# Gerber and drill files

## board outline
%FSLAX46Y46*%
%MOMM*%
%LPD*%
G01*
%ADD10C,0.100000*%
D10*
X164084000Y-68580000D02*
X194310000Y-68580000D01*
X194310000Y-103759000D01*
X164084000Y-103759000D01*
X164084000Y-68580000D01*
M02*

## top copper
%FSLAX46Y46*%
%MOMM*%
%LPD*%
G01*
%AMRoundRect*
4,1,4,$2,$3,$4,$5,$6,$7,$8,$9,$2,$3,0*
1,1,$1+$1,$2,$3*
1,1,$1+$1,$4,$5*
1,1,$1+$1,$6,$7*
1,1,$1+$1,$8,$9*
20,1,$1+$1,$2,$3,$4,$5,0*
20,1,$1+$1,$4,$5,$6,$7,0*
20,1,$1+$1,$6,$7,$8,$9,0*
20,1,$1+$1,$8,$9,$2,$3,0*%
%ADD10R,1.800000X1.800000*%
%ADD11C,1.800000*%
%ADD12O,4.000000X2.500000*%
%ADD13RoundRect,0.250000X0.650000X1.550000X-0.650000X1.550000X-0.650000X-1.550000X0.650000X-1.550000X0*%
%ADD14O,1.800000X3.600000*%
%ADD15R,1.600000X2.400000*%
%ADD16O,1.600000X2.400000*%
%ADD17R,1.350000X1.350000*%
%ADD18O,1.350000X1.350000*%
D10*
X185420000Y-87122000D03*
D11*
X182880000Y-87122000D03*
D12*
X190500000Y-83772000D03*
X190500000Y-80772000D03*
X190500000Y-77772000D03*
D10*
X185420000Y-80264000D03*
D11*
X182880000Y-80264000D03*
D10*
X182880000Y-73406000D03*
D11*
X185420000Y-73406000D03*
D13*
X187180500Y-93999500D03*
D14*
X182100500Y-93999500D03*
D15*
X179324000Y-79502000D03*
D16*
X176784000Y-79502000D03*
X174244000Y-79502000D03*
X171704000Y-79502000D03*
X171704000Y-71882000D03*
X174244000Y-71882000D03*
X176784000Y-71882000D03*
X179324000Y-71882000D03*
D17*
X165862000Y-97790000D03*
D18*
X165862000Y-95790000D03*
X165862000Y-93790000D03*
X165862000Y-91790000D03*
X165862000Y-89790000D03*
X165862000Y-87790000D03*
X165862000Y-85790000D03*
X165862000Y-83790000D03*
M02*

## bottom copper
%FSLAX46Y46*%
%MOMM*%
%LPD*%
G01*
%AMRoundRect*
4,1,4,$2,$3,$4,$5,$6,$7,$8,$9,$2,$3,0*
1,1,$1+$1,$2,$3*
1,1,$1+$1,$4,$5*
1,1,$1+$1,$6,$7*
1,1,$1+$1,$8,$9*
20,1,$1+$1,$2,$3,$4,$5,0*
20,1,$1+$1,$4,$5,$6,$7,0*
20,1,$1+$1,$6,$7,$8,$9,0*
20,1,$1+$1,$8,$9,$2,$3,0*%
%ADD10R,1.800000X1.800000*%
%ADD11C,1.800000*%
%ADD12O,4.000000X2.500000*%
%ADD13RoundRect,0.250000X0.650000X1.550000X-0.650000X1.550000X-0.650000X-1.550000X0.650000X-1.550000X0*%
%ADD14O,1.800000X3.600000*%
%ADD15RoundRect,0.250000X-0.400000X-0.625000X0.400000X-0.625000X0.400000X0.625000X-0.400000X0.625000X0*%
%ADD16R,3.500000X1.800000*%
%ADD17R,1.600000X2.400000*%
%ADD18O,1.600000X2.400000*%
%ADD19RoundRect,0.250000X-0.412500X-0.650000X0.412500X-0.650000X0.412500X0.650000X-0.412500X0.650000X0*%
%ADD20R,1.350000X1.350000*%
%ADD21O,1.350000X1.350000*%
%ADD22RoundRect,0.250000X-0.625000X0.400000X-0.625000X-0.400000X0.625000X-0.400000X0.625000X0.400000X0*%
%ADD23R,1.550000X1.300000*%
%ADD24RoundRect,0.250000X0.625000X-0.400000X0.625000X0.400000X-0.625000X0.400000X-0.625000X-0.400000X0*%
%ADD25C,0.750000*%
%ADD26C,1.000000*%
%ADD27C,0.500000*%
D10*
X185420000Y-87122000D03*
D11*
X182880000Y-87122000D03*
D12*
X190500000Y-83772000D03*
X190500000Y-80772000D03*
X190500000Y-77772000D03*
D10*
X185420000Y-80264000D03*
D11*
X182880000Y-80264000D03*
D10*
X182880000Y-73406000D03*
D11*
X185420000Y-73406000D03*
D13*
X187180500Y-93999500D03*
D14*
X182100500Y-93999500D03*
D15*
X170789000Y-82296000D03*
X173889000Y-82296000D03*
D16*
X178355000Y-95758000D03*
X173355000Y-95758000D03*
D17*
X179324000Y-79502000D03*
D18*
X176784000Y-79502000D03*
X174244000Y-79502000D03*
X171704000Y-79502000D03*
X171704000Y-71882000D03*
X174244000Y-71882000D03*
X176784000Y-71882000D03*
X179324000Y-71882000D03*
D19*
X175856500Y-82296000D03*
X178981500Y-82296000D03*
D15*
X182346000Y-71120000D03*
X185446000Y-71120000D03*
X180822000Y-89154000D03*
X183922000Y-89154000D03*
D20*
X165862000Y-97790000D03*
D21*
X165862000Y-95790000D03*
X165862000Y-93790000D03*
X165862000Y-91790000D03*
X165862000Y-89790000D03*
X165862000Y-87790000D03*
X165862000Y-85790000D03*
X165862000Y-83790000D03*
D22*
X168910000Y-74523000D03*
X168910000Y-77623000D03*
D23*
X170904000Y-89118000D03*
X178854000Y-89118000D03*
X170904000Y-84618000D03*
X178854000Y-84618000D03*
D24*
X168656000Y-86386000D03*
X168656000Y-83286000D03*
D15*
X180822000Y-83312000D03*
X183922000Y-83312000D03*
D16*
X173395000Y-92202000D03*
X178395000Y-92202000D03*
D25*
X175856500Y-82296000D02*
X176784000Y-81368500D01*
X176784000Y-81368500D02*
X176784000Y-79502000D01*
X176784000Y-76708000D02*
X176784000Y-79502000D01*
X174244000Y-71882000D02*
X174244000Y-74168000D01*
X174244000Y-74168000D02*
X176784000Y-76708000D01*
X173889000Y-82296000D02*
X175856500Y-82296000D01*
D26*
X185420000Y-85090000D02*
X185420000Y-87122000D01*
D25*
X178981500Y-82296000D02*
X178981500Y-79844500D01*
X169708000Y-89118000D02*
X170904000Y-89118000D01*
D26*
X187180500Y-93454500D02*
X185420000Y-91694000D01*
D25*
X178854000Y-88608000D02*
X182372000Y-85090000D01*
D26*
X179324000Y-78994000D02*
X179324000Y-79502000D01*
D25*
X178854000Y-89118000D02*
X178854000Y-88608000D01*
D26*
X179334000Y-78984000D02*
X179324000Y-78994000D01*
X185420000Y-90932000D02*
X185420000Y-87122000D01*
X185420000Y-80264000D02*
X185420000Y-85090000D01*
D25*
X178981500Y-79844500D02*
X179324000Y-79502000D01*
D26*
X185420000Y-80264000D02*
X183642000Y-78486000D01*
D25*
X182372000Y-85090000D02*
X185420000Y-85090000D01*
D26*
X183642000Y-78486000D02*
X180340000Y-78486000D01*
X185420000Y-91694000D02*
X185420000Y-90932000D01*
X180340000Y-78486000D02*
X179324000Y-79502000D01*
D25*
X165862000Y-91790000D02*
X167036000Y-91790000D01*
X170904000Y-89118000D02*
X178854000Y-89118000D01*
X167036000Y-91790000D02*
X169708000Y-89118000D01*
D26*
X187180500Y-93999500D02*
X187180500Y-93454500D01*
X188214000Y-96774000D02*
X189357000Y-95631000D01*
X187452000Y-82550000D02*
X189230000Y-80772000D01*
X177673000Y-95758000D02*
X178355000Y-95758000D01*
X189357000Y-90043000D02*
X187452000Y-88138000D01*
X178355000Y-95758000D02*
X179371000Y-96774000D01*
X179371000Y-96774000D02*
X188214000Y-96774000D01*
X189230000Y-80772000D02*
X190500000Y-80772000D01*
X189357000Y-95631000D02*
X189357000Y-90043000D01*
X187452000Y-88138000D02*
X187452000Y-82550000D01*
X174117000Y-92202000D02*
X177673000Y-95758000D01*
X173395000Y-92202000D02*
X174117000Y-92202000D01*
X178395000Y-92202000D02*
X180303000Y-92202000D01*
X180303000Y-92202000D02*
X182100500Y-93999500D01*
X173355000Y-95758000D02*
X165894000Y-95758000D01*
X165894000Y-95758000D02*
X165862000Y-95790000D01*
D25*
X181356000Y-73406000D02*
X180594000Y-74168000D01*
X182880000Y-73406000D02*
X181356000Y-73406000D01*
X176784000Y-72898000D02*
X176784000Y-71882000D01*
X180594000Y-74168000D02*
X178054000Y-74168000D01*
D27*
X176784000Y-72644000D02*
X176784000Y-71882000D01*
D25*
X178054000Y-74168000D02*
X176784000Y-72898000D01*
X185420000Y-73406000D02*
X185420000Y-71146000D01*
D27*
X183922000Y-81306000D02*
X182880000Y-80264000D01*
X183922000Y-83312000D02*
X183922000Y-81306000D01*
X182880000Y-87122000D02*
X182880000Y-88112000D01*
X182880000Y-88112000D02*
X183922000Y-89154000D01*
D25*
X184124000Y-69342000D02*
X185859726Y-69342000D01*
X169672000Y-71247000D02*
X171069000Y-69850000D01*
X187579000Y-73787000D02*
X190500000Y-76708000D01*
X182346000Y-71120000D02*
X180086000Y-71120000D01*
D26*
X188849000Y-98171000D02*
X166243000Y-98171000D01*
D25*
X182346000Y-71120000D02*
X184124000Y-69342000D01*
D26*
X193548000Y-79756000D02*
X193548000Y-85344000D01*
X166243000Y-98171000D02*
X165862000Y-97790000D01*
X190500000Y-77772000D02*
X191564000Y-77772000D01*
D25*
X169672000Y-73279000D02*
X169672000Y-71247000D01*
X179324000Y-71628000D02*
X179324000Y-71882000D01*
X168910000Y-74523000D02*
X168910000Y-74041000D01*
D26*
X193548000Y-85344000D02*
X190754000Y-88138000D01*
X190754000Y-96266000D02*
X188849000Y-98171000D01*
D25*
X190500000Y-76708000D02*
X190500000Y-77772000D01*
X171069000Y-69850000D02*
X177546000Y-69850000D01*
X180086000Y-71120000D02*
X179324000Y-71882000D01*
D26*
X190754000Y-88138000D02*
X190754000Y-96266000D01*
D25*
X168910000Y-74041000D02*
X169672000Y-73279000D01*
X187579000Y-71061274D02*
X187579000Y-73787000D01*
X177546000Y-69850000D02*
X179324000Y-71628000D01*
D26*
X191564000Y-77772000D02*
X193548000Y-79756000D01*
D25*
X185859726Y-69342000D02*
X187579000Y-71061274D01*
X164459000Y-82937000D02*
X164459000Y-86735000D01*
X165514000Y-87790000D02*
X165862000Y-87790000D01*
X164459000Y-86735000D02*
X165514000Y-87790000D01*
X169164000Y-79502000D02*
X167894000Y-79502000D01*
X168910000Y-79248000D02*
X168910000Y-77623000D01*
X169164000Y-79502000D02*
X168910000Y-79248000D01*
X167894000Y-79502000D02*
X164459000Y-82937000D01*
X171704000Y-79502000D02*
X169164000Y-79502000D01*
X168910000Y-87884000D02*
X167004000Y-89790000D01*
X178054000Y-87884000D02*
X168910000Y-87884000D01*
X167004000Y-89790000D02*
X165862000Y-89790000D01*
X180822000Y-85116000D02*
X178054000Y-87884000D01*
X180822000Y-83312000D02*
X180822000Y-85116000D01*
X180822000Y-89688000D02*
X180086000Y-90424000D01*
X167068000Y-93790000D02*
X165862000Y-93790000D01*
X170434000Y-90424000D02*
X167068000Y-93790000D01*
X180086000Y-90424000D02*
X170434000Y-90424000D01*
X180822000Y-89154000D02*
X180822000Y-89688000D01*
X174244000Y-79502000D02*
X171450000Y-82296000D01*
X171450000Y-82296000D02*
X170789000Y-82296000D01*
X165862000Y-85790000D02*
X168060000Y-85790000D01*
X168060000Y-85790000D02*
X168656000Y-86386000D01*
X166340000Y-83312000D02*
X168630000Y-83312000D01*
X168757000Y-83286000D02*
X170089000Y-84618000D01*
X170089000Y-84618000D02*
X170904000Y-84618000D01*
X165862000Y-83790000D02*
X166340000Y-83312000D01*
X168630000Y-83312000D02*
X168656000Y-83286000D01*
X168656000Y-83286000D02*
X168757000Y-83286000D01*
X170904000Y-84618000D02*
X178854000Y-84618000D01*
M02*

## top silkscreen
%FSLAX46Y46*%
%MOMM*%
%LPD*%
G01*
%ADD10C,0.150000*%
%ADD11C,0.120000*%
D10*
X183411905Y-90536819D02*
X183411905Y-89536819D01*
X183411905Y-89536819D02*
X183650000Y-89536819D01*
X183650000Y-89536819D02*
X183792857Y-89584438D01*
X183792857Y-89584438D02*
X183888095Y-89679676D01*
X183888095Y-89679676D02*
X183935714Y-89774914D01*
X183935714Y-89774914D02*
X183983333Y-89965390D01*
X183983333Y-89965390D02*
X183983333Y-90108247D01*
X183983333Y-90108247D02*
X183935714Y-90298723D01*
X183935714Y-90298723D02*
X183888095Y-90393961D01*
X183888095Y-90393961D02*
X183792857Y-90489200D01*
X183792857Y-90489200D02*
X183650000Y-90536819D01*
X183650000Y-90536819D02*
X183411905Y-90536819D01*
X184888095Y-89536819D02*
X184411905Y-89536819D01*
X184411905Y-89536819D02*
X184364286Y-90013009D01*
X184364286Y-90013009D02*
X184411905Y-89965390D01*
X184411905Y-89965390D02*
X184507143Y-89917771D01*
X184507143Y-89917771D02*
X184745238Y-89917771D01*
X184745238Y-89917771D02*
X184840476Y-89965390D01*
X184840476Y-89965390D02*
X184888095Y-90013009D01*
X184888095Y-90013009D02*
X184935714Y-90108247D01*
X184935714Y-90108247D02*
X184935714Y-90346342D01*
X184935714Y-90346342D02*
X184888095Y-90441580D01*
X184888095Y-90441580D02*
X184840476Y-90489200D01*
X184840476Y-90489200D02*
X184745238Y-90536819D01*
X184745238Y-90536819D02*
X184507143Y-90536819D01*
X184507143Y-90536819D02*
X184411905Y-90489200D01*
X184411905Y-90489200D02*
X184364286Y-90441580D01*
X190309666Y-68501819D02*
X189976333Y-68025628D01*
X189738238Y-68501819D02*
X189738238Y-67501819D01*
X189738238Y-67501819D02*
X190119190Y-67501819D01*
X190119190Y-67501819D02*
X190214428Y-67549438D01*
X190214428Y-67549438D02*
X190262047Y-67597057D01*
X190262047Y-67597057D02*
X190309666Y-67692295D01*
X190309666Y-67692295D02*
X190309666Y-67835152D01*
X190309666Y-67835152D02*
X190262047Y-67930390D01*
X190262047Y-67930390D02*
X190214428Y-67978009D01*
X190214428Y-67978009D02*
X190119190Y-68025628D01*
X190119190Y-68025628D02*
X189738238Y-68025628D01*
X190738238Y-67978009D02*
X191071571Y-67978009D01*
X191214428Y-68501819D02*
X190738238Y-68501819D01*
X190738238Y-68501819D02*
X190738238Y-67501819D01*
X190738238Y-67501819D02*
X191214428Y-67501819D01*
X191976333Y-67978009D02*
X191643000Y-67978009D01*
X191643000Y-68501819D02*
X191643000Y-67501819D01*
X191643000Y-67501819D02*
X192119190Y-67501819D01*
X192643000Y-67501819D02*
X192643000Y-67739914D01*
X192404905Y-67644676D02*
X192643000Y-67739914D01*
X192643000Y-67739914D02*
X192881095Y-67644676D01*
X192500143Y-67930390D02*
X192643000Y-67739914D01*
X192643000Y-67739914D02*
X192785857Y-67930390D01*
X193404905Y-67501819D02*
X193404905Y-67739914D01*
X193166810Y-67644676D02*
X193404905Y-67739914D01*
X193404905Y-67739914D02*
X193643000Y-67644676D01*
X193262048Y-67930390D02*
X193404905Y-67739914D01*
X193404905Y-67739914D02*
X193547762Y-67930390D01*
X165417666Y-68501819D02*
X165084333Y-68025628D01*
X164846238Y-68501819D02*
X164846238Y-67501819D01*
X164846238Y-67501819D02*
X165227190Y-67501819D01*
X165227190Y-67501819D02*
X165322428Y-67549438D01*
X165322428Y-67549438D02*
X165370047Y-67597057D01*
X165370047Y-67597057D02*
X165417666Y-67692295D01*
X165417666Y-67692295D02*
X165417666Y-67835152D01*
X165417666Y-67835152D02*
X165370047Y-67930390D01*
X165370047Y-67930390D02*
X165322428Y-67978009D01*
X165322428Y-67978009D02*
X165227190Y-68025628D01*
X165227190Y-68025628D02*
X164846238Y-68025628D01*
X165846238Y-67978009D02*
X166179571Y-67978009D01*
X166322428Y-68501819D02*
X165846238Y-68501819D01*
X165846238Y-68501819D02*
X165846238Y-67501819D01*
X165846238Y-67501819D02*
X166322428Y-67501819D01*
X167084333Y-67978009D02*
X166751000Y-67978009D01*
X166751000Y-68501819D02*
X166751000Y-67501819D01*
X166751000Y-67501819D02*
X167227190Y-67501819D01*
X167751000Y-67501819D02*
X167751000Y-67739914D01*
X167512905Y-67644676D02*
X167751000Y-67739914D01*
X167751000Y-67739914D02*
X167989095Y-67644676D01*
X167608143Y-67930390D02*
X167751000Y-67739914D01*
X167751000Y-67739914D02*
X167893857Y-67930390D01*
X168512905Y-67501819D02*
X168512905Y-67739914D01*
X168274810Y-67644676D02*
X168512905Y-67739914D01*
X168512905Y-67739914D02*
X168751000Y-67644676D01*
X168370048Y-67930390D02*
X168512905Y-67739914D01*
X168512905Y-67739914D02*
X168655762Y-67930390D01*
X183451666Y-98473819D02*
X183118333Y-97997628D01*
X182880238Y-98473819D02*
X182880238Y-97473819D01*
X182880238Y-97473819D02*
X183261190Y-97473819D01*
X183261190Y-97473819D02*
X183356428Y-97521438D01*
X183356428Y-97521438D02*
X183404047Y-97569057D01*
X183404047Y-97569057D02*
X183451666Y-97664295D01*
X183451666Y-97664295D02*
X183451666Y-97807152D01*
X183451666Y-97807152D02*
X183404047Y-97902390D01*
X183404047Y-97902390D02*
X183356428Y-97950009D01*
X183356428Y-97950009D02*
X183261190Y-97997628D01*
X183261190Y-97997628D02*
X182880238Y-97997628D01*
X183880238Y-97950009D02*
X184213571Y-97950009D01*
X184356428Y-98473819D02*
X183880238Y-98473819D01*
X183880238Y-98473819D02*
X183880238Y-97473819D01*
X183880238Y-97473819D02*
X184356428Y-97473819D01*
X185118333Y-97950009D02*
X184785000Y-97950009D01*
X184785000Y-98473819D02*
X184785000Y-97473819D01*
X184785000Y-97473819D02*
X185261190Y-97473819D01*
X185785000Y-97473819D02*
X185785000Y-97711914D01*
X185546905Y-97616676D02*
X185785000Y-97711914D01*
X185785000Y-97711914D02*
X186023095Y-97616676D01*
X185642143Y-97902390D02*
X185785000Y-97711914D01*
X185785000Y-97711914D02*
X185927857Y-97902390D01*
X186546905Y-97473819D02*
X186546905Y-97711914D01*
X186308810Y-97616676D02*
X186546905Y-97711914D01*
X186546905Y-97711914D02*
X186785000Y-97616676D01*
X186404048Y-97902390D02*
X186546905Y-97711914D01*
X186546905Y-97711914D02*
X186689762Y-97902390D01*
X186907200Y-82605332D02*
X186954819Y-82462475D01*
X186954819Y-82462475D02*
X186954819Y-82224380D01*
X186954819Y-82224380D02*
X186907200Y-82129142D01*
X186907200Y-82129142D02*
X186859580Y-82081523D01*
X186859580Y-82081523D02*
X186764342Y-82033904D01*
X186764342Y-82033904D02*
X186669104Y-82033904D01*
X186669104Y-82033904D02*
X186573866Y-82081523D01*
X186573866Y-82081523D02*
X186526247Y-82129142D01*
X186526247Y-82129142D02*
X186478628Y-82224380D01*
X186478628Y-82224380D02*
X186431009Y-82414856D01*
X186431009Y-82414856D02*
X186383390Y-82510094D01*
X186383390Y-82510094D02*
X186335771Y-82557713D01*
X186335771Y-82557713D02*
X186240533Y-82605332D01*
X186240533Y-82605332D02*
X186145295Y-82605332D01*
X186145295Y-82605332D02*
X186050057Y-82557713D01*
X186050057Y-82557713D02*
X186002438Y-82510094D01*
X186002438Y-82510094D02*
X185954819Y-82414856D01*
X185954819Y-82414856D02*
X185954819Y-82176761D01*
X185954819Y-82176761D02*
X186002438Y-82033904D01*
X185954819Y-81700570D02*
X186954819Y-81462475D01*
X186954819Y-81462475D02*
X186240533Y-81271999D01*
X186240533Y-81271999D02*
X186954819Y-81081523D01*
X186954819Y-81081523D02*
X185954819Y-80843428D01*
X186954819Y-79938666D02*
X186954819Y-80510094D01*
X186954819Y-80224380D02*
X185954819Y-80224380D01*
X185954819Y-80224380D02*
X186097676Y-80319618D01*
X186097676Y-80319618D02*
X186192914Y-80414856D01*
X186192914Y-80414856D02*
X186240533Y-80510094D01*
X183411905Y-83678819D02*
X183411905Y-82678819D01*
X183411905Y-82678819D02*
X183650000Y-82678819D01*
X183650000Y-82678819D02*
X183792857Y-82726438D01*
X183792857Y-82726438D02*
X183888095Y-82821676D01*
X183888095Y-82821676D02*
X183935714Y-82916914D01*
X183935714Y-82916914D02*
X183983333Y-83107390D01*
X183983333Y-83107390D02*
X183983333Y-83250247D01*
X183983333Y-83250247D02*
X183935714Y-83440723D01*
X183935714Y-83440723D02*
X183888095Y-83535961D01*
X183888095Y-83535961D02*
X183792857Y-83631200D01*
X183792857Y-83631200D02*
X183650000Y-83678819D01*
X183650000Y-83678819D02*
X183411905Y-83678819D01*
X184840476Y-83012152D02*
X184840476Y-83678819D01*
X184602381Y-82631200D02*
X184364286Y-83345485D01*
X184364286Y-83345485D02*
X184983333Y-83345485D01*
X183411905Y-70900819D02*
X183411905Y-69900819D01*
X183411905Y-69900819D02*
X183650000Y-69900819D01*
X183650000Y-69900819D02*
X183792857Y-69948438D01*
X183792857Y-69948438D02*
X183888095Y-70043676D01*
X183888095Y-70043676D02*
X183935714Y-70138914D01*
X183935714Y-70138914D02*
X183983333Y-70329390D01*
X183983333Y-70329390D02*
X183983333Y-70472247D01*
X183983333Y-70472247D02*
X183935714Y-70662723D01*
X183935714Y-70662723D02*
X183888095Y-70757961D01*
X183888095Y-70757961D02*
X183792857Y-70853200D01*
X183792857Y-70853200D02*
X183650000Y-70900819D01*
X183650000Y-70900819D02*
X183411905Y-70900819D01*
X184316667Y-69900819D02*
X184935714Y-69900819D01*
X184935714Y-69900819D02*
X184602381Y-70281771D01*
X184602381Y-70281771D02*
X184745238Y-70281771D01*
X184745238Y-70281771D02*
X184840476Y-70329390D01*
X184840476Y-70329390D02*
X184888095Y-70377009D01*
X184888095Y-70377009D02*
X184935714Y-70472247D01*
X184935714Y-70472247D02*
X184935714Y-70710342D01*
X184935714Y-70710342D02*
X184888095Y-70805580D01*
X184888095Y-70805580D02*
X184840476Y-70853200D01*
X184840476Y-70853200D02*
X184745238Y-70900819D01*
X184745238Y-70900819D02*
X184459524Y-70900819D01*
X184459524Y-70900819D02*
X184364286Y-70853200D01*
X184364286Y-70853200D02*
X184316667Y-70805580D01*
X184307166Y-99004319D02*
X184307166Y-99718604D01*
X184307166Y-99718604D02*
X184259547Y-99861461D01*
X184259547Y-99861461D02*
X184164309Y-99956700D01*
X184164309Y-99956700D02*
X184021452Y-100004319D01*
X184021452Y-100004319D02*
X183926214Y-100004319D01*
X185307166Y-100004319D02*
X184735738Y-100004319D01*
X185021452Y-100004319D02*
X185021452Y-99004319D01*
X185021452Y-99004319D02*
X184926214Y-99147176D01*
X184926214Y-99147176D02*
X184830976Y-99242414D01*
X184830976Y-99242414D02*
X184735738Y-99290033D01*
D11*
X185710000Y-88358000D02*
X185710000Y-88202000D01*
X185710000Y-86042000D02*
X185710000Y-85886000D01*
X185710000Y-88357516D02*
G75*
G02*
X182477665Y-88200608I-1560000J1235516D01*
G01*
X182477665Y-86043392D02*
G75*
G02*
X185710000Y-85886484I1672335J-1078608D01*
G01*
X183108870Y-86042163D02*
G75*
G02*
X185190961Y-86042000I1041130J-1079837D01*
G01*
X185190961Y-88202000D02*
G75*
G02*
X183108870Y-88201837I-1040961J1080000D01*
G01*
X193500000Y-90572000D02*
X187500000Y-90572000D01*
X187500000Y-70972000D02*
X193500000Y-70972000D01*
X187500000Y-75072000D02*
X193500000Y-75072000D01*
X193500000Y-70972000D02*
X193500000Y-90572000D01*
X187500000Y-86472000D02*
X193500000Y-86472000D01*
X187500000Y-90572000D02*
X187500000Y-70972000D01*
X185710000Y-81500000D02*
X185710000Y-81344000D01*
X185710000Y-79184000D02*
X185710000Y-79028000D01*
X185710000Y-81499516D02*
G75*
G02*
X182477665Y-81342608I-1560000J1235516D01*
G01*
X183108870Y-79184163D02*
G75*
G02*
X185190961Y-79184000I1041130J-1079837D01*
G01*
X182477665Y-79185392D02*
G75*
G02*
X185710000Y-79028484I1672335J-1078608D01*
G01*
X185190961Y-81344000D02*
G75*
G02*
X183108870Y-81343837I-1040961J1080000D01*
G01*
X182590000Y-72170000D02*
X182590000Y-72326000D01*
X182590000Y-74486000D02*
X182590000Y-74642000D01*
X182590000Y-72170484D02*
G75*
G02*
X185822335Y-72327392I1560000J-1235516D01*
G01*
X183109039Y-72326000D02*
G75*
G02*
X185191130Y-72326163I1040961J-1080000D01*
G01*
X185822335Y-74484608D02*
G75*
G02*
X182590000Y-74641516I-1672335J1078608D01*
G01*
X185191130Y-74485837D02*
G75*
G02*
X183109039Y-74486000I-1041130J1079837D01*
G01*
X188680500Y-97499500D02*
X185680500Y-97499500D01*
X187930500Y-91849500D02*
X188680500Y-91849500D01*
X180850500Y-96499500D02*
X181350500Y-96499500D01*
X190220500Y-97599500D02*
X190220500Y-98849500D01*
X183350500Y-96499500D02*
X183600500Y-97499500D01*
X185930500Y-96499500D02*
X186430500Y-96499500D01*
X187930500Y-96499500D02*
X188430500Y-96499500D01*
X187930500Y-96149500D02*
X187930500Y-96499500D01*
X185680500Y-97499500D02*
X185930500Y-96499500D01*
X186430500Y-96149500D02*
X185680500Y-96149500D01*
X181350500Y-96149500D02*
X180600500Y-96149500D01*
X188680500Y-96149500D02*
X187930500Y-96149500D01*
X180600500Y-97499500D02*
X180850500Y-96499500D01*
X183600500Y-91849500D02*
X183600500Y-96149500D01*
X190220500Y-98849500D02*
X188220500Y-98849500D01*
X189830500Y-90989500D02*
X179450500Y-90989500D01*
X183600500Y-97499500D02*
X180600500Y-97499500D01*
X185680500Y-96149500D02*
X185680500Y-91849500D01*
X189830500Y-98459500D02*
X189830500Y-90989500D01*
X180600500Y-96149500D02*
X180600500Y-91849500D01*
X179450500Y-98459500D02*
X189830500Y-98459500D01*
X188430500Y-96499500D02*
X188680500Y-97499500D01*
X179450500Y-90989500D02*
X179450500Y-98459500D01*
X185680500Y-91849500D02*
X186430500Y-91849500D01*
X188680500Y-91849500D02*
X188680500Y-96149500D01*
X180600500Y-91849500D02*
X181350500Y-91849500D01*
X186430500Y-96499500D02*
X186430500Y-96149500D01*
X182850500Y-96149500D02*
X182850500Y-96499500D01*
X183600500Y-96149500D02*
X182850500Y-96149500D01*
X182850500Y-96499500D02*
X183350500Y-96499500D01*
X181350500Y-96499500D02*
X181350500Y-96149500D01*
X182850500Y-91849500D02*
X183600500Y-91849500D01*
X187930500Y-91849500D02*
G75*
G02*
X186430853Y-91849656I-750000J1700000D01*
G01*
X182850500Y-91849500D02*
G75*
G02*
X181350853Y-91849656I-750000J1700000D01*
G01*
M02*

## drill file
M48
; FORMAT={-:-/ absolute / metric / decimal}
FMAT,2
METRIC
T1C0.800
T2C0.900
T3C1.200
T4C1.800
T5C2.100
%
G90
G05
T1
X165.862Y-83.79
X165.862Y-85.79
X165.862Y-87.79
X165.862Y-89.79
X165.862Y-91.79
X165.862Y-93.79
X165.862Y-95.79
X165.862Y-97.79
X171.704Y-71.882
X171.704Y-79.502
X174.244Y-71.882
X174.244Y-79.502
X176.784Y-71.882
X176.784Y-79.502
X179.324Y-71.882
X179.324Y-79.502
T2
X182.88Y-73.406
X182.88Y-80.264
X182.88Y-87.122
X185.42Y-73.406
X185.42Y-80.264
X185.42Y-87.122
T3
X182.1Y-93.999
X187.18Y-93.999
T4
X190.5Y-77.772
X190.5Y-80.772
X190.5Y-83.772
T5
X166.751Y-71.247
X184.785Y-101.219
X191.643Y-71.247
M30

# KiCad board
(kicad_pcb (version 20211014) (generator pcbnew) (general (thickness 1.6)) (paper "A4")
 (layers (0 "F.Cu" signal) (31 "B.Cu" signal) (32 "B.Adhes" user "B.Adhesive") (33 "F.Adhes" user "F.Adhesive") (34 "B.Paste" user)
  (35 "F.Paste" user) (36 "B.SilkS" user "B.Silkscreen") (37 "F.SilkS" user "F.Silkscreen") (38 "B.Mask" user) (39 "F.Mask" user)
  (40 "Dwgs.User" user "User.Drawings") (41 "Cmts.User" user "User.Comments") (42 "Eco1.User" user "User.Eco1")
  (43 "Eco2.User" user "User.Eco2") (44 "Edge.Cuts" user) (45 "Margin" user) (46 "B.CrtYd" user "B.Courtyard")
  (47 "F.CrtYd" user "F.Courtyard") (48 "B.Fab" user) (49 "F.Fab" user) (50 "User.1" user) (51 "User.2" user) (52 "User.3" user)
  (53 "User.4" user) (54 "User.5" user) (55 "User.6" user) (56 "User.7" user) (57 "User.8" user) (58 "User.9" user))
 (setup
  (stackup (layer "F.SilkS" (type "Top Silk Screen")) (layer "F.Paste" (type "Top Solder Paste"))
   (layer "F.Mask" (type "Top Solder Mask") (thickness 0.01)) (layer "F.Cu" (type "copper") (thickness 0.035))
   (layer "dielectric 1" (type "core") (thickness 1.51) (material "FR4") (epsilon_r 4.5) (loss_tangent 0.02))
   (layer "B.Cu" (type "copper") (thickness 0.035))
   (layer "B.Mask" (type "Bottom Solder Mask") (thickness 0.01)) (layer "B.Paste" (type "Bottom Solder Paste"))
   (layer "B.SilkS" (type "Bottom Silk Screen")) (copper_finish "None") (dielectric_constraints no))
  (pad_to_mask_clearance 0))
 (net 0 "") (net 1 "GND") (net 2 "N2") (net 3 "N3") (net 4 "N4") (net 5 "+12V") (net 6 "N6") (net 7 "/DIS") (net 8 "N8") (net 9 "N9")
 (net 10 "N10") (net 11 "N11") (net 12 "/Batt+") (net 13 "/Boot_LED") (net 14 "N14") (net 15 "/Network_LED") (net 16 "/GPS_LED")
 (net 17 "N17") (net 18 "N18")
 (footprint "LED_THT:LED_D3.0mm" (layer "F.Cu") (at 185.42 87.122 180)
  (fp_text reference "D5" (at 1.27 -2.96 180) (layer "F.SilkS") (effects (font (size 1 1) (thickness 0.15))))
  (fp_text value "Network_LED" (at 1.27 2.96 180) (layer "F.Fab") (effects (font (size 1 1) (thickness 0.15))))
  (fp_line (start -0.29 -1.236) (end -0.29 -1.08) (layer "F.SilkS") (width 0.12))
  (fp_line (start -0.29 1.08) (end -0.29 1.236) (layer "F.SilkS") (width 0.12))
  (fp_arc (start -0.29 -1.235516) (mid 1.366487 -1.987659) (end 2.942335 -1.078608) (layer "F.SilkS") (width 0.12))
  (fp_arc (start 2.942335 1.078608) (mid 1.366487 1.987659) (end -0.29 1.235516) (layer "F.SilkS") (width 0.12))
  (fp_arc (start 2.31113 1.079837) (mid 1.270117 1.5) (end 0.229039 1.08) (layer "F.SilkS") (width 0.12))
  (fp_arc (start 0.229039 -1.08) (mid 1.270117 -1.5) (end 2.31113 -1.079837) (layer "F.SilkS") (width 0.12))
  (pad "1" thru_hole rect (at 0 0 180) (size 1.8 1.8) (drill 0.9) (layers *.Cu *.Mask) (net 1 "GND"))
  (pad "2" thru_hole circle (at 2.54 0 180) (size 1.8 1.8) (drill 0.9) (layers *.Cu *.Mask) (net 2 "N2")))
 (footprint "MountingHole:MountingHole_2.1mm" (layer "F.Cu") (at 191.643 71.247)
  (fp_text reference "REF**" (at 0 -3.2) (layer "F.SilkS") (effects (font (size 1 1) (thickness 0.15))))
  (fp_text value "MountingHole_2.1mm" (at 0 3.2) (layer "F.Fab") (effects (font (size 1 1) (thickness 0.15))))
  (pad "" np_thru_hole circle (at 0 0) (size 2.1 2.1) (drill 2.1) (layers *.Cu *.Mask)))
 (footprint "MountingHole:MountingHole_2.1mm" (layer "F.Cu") (at 166.751 71.247)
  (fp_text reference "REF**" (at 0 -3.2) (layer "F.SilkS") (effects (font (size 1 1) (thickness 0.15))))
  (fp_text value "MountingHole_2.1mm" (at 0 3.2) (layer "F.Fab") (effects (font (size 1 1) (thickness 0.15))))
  (pad "" np_thru_hole circle (at 0 0) (size 2.1 2.1) (drill 2.1) (layers *.Cu *.Mask)))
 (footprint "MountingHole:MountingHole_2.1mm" (layer "F.Cu") (at 184.785 101.219)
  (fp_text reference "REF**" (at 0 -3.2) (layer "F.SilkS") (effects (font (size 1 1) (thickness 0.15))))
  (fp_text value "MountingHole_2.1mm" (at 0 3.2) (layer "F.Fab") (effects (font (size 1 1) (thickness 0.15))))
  (pad "" np_thru_hole circle (at 0 0) (size 2.1 2.1) (drill 2.1) (layers *.Cu *.Mask)))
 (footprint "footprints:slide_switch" (layer "F.Cu") (at 190.5 80.772 90) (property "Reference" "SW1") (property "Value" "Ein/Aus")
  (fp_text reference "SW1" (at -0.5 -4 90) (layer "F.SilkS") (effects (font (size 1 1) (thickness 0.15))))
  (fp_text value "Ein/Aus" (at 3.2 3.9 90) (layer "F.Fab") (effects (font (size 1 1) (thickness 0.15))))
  (fp_line (start -9.8 3) (end -9.8 -3) (layer "F.SilkS") (width 0.12))
  (fp_line (start 9.8 -3) (end 9.8 3) (layer "F.SilkS") (width 0.12))
  (fp_line (start 5.7 -3) (end 5.7 3) (layer "F.SilkS") (width 0.12))
  (fp_line (start 9.8 3) (end -9.8 3) (layer "F.SilkS") (width 0.12))
  (fp_line (start -5.7 -3) (end -5.7 3) (layer "F.SilkS") (width 0.12))
  (fp_line (start -9.8 -3) (end 9.8 -3) (layer "F.SilkS") (width 0.12))
  (pad "1" thru_hole oval (at -3 0 90) (size 2.5 4) (drill 1.8) (layers *.Cu *.Mask) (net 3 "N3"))
  (pad "2" thru_hole oval (at 0 0 90) (size 2.5 4) (drill 1.8) (layers *.Cu *.Mask) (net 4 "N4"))
  (pad "3" thru_hole oval (at 3 0 90) (size 2.5 4) (drill 1.8) (layers *.Cu *.Mask) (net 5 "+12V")))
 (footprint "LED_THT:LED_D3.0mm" (layer "F.Cu") (at 185.42 80.264 180) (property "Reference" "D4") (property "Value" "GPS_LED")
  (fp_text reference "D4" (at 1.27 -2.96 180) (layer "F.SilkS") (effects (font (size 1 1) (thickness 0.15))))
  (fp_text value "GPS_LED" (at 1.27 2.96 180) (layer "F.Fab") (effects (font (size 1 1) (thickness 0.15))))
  (fp_line (start -0.29 -1.236) (end -0.29 -1.08) (layer "F.SilkS") (width 0.12))
  (fp_line (start -0.29 1.08) (end -0.29 1.236) (layer "F.SilkS") (width 0.12))
  (fp_arc (start -0.29 -1.235516) (mid 1.366487 -1.987659) (end 2.942335 -1.078608) (layer "F.SilkS") (width 0.12))
  (fp_arc (start 2.31113 1.079837) (mid 1.270117 1.5) (end 0.229039 1.08) (layer "F.SilkS") (width 0.12))
  (fp_arc (start 2.942335 1.078608) (mid 1.366487 1.987659) (end -0.29 1.235516) (layer "F.SilkS") (width 0.12))
  (fp_arc (start 0.229039 -1.08) (mid 1.270117 -1.5) (end 2.31113 -1.079837) (layer "F.SilkS") (width 0.12))
  (pad "1" thru_hole rect (at 0 0 180) (size 1.8 1.8) (drill 0.9) (layers *.Cu *.Mask) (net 1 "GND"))
  (pad "2" thru_hole circle (at 2.54 0 180) (size 1.8 1.8) (drill 0.9) (layers *.Cu *.Mask) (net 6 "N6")))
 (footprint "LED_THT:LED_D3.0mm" (layer "F.Cu") (at 182.88 73.406)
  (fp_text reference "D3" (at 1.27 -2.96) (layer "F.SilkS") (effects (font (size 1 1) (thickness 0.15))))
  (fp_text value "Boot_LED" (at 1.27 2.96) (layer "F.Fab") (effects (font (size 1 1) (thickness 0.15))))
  (fp_line (start -0.29 -1.236) (end -0.29 -1.08) (layer "F.SilkS") (width 0.12))
  (fp_line (start -0.29 1.08) (end -0.29 1.236) (layer "F.SilkS") (width 0.12))
  (fp_arc (start -0.29 -1.235516) (mid 1.366487 -1.987659) (end 2.942335 -1.078608) (layer "F.SilkS") (width 0.12))
  (fp_arc (start 0.229039 -1.08) (mid 1.270117 -1.5) (end 2.31113 -1.079837) (layer "F.SilkS") (width 0.12))
  (fp_arc (start 2.942335 1.078608) (mid 1.366487 1.987659) (end -0.29 1.235516) (layer "F.SilkS") (width 0.12))
  (fp_arc (start 2.31113 1.079837) (mid 1.270117 1.5) (end 0.229039 1.08) (layer "F.SilkS") (width 0.12))
  (pad "1" thru_hole rect (at 0 0) (size 1.8 1.8) (drill 0.9) (layers *.Cu *.Mask) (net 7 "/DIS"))
  (pad "2" thru_hole circle (at 2.54 0) (size 1.8 1.8) (drill 0.9) (layers *.Cu *.Mask) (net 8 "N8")))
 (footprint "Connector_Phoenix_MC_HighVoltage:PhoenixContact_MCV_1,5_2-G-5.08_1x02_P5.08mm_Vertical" (layer "F.Cu")
  (at 187.1805 93.9995 180) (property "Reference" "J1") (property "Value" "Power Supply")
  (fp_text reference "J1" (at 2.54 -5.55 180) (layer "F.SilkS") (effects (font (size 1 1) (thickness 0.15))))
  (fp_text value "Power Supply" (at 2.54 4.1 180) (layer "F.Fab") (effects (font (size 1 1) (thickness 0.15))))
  (fp_line (start -1.5 -3.5) (end 1.5 -3.5) (layer "F.SilkS") (width 0.12))
  (fp_line (start -0.75 2.15) (end -1.5 2.15) (layer "F.SilkS") (width 0.12))
  (fp_line (start 6.33 -2.5) (end 5.83 -2.5) (layer "F.SilkS") (width 0.12))
  (fp_line (start -3.04 -3.6) (end -3.04 -4.85) (layer "F.SilkS") (width 0.12))
  (fp_line (start 3.83 -2.5) (end 3.58 -3.5) (layer "F.SilkS") (width 0.12))
  (fp_line (start 1.25 -2.5) (end 0.75 -2.5) (layer "F.SilkS") (width 0.12))
  (fp_line (start -0.75 -2.5) (end -1.25 -2.5) (layer "F.SilkS") (width 0.12))
  (fp_line (start -0.75 -2.15) (end -0.75 -2.5) (layer "F.SilkS") (width 0.12))
  (fp_line (start 1.5 -3.5) (end 1.25 -2.5) (layer "F.SilkS") (width 0.12))
  (fp_line (start 0.75 -2.15) (end 1.5 -2.15) (layer "F.SilkS") (width 0.12))
  (fp_line (start 5.83 -2.15) (end 6.58 -2.15) (layer "F.SilkS") (width 0.12))
  (fp_line (start -1.5 -2.15) (end -0.75 -2.15) (layer "F.SilkS") (width 0.12))
  (fp_line (start 6.58 -3.5) (end 6.33 -2.5) (layer "F.SilkS") (width 0.12))
  (fp_line (start 3.58 2.15) (end 3.58 -2.15) (layer "F.SilkS") (width 0.12))
  (fp_line (start -3.04 -4.85) (end -1.04 -4.85) (layer "F.SilkS") (width 0.12))
  (fp_line (start -2.65 3.01) (end 7.73 3.01) (layer "F.SilkS") (width 0.12))
  (fp_line (start 3.58 -3.5) (end 6.58 -3.5) (layer "F.SilkS") (width 0.12))
  (fp_line (start 1.5 -2.15) (end 1.5 2.15) (layer "F.SilkS") (width 0.12))
  (fp_line (start -2.65 -4.46) (end -2.65 3.01) (layer "F.SilkS") (width 0.12))
  (fp_line (start 6.58 -2.15) (end 6.58 2.15) (layer "F.SilkS") (width 0.12))
  (fp_line (start 7.73 -4.46) (end -2.65 -4.46) (layer "F.SilkS") (width 0.12))
  (fp_line (start -1.25 -2.5) (end -1.5 -3.5) (layer "F.SilkS") (width 0.12))
  (fp_line (start 7.73 3.01) (end 7.73 -4.46) (layer "F.SilkS") (width 0.12))
  (fp_line (start 1.5 2.15) (end 0.75 2.15) (layer "F.SilkS") (width 0.12))
  (fp_line (start -1.5 2.15) (end -1.5 -2.15) (layer "F.SilkS") (width 0.12))
  (fp_line (start 6.58 2.15) (end 5.83 2.15) (layer "F.SilkS") (width 0.12))
  (fp_line (start 0.75 -2.5) (end 0.75 -2.15) (layer "F.SilkS") (width 0.12))
  (fp_line (start 4.33 -2.15) (end 4.33 -2.5) (layer "F.SilkS") (width 0.12))
  (fp_line (start 3.58 -2.15) (end 4.33 -2.15) (layer "F.SilkS") (width 0.12))
  (fp_line (start 4.33 -2.5) (end 3.83 -2.5) (layer "F.SilkS") (width 0.12))
  (fp_line (start 5.83 -2.5) (end 5.83 -2.15) (layer "F.SilkS") (width 0.12))
  (fp_line (start 4.33 2.15) (end 3.58 2.15) (layer "F.SilkS") (width 0.12))
  (fp_arc (start -0.75 2.15) (mid -0.000193 1.99191) (end 0.749647 2.149844) (layer "F.SilkS") (width 0.12))
  (fp_arc (start 4.33 2.15) (mid 5.079807 1.99191) (end 5.829647 2.149844) (layer "F.SilkS") (width 0.12))
  (pad "1" thru_hole roundrect (at 0 0 180) (size 1.8 3.6) (drill 1.2) (layers *.Cu *.Mask) (roundrect_rratio 0.1388888889) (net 1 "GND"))
  (pad "2" thru_hole oval (at 5.08 0 180) (size 1.8 3.6) (drill 1.2) (layers *.Cu *.Mask) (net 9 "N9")))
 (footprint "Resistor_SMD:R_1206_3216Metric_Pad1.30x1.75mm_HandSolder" (layer "B.Cu") (at 172.339 82.296) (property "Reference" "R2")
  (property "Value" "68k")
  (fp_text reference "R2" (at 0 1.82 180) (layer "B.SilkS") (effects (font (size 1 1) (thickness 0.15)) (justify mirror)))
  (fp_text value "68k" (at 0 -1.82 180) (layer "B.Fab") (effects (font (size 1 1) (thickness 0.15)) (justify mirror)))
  (pad "1" smd roundrect (at -1.55 0) (size 1.3 1.75) (layers "B.Cu" "B.Paste" "B.Mask") (roundrect_rratio 0.1923076923) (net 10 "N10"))
  (pad "2" smd roundrect (at 1.55 0) (size 1.3 1.75) (layers "B.Cu" "B.Paste" "B.Mask") (roundrect_rratio 0.1923076923) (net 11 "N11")))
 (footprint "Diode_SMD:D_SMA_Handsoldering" (layer "B.Cu") (at 175.855 95.758 180) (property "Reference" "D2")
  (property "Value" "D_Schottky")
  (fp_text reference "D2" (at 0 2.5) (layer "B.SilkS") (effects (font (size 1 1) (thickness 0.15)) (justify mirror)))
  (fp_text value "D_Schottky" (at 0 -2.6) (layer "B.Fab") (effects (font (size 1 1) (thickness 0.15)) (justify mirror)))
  (pad "1" smd rect (at -2.5 0 180) (size 3.5 1.8) (layers "B.Cu" "B.Paste" "B.Mask") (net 4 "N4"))
  (pad "2" smd rect (at 2.5 0 180) (size 3.5 1.8) (layers "B.Cu" "B.Paste" "B.Mask") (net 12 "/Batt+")))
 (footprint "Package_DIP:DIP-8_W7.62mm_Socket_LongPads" (layer "B.Cu") (at 179.324 79.502 90) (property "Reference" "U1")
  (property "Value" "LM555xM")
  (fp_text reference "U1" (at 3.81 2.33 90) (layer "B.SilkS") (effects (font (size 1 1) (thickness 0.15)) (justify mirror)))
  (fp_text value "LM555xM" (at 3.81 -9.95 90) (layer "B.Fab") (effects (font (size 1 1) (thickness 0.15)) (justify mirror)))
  (pad "1" thru_hole rect (at 0 0 90) (size 2.4 1.6) (drill 0.8) (layers *.Cu *.Mask) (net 1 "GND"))
  (pad "2" thru_hole oval (at 0 -2.54 90) (size 2.4 1.6) (drill 0.8) (layers *.Cu *.Mask) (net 11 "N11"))
  (pad "3" thru_hole oval (at 0 -5.08 90) (size 2.4 1.6) (drill 0.8) (layers *.Cu *.Mask) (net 10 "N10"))
  (pad "4" thru_hole oval (at 0 -7.62 90) (size 2.4 1.6) (drill 0.8) (layers *.Cu *.Mask) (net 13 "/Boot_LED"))
  (pad "5" thru_hole oval (at 7.62 -7.62 90) (size 2.4 1.6) (drill 0.8) (layers *.Cu *.Mask) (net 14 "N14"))
  (pad "6" thru_hole oval (at 7.62 -5.08 90) (size 2.4 1.6) (drill 0.8) (layers *.Cu *.Mask) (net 11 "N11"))
  (pad "7" thru_hole oval (at 7.62 -2.54 90) (size 2.4 1.6) (drill 0.8) (layers *.Cu *.Mask) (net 7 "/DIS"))
  (pad "8" thru_hole oval (at 7.62 0 90) (size 2.4 1.6) (drill 0.8) (layers *.Cu *.Mask) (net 5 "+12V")))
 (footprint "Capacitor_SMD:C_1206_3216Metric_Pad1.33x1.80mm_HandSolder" (layer "B.Cu") (at 177.419 82.296) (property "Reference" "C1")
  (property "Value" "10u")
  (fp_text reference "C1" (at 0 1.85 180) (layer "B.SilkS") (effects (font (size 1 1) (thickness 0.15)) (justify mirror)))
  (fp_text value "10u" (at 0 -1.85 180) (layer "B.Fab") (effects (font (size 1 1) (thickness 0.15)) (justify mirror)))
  (pad "1" smd roundrect (at -1.5625 0) (size 1.325 1.8) (layers "B.Cu" "B.Paste" "B.Mask") (roundrect_rratio 0.1886792453) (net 11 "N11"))
  (pad "2" smd roundrect (at 1.5625 0) (size 1.325 1.8) (layers "B.Cu" "B.Paste" "B.Mask") (roundrect_rratio 0.1886792453) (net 1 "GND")))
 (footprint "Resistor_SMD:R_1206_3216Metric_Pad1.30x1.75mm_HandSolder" (layer "B.Cu") (at 183.896 71.12)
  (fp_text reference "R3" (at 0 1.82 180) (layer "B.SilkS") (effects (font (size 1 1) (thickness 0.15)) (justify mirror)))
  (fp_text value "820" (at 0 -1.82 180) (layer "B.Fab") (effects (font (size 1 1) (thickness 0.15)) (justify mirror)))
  (pad "1" smd roundrect (at -1.55 0) (size 1.3 1.75) (layers "B.Cu" "B.Paste" "B.Mask") (roundrect_rratio 0.1923076923) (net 5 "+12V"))
  (pad "2" smd roundrect (at 1.55 0) (size 1.3 1.75) (layers "B.Cu" "B.Paste" "B.Mask") (roundrect_rratio 0.1923076923) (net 8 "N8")))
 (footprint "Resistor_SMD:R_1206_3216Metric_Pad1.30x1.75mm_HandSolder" (layer "B.Cu") (at 182.372 89.154)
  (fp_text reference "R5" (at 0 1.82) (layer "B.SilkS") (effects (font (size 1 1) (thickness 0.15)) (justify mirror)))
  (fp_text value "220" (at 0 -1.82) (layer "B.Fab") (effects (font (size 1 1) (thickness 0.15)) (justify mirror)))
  (pad "1" smd roundrect (at -1.55 0) (size 1.3 1.75) (layers "B.Cu" "B.Paste" "B.Mask") (roundrect_rratio 0.1923076923)
   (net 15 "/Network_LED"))
  (pad "2" smd roundrect (at 1.55 0) (size 1.3 1.75) (layers "B.Cu" "B.Paste" "B.Mask") (roundrect_rratio 0.1923076923) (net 2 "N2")))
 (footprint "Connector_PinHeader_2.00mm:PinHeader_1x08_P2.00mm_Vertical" (layer "B.Cu") (at 165.862 97.79)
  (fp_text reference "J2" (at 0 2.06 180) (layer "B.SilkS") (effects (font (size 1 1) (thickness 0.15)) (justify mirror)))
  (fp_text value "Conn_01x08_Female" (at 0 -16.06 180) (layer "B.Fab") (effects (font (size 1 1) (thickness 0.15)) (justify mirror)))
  (pad "1" thru_hole rect (at 0 0) (size 1.35 1.35) (drill 0.8) (layers *.Cu *.Mask) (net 5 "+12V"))
  (pad "2" thru_hole oval (at 0 -2) (size 1.35 1.35) (drill 0.8) (layers *.Cu *.Mask) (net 12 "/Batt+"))
  (pad "3" thru_hole oval (at 0 -4) (size 1.35 1.35) (drill 0.8) (layers *.Cu *.Mask) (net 15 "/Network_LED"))
  (pad "4" thru_hole oval (at 0 -6) (size 1.35 1.35) (drill 0.8) (layers *.Cu *.Mask) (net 1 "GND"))
  (pad "5" thru_hole oval (at 0 -8) (size 1.35 1.35) (drill 0.8) (layers *.Cu *.Mask) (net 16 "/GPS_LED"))
  (pad "6" thru_hole oval (at 0 -10) (size 1.35 1.35) (drill 0.8) (layers *.Cu *.Mask) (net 13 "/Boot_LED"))
  (pad "7" thru_hole oval (at 0 -12) (size 1.35 1.35) (drill 0.8) (layers *.Cu *.Mask) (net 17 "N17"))
  (pad "8" thru_hole oval (at 0 -14) (size 1.35 1.35) (drill 0.8) (layers *.Cu *.Mask) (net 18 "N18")))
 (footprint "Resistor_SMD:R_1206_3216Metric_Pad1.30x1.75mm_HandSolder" (layer "B.Cu") (at 168.91 76.073 -90)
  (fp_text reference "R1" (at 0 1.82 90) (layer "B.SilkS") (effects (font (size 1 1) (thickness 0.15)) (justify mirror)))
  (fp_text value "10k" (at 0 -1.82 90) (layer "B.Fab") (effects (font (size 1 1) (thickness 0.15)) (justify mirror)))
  (pad "1" smd roundrect (at -1.55 0 270) (size 1.3 1.75) (layers "B.Cu" "B.Paste" "B.Mask") (roundrect_rratio 0.1923076923) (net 5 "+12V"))
  (pad "2" smd roundrect (at 1.55 0 270) (size 1.3 1.75) (layers "B.Cu" "B.Paste" "B.Mask") (roundrect_rratio 0.1923076923)
   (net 13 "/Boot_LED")))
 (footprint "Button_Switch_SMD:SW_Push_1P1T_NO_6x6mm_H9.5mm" (layer "B.Cu") (at 174.879 86.868)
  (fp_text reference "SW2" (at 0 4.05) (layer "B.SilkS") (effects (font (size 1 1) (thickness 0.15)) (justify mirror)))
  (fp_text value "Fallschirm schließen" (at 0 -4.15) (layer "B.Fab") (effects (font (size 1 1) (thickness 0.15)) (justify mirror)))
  (pad "1" smd rect (at -3.975 2.25) (size 1.55 1.3) (layers "B.Cu" "B.Paste" "B.Mask") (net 1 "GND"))
  (pad "1" smd rect (at 3.975 2.25) (size 1.55 1.3) (layers "B.Cu" "B.Paste" "B.Mask") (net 1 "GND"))
  (pad "2" smd rect (at -3.975 -2.25) (size 1.55 1.3) (layers "B.Cu" "B.Paste" "B.Mask") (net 18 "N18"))
  (pad "2" smd rect (at 3.975 -2.25) (size 1.55 1.3) (layers "B.Cu" "B.Paste" "B.Mask") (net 18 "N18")))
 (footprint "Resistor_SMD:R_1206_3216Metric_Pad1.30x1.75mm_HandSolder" (layer "B.Cu") (at 168.656 84.836 90)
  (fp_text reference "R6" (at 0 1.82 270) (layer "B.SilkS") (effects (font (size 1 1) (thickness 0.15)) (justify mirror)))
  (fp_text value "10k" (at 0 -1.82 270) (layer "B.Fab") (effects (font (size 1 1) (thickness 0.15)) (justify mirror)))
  (pad "1" smd roundrect (at -1.55 0 90) (size 1.3 1.75) (layers "B.Cu" "B.Paste" "B.Mask") (roundrect_rratio 0.1923076923) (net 17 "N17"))
  (pad "2" smd roundrect (at 1.55 0 90) (size 1.3 1.75) (layers "B.Cu" "B.Paste" "B.Mask") (roundrect_rratio 0.1923076923) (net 18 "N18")))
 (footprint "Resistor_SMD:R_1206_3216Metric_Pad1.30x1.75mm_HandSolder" (layer "B.Cu") (at 182.372 83.312) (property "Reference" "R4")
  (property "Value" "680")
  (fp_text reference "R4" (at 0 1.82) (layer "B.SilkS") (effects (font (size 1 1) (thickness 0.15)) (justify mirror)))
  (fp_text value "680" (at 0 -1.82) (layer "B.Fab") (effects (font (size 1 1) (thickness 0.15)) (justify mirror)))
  (pad "1" smd roundrect (at -1.55 0) (size 1.3 1.75) (layers "B.Cu" "B.Paste" "B.Mask") (roundrect_rratio 0.1923076923) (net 16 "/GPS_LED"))
  (pad "2" smd roundrect (at 1.55 0) (size 1.3 1.75) (layers "B.Cu" "B.Paste" "B.Mask") (roundrect_rratio 0.1923076923) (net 6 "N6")))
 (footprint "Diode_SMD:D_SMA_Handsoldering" (layer "B.Cu") (at 175.895 92.202) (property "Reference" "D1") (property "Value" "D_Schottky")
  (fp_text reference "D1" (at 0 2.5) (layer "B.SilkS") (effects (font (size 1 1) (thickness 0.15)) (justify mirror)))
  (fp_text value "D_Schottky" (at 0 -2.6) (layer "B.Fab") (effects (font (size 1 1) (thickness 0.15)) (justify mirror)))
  (pad "1" smd rect (at -2.5 0) (size 3.5 1.8) (layers "B.Cu" "B.Paste" "B.Mask") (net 4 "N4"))
  (pad "2" smd rect (at 2.5 0) (size 3.5 1.8) (layers "B.Cu" "B.Paste" "B.Mask") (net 9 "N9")))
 (gr_rect (start 164.084 68.58) (end 194.31 103.759) (layer "Edge.Cuts") (width 0.1) (fill none))
 (segment (start 175.8565 82.296) (end 176.784 81.3685) (width 0.75) (layer "B.Cu") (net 11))
 (segment (start 176.784 81.3685) (end 176.784 79.502) (width 0.75) (layer "B.Cu") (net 11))
 (segment (start 176.784 76.708) (end 176.784 79.502) (width 0.75) (layer "B.Cu") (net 11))
 (segment (start 174.244 71.882) (end 174.244 74.168) (width 0.75) (layer "B.Cu") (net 11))
 (segment (start 174.244 74.168) (end 176.784 76.708) (width 0.75) (layer "B.Cu") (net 11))
 (segment (start 173.889 82.296) (end 175.8565 82.296) (width 0.75) (layer "B.Cu") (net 11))
 (segment (start 185.42 85.09) (end 185.42 87.122) (width 1) (layer "B.Cu") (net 1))
 (segment (start 178.9815 82.296) (end 178.9815 79.8445) (width 0.75) (layer "B.Cu") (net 1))
 (segment (start 169.708 89.118) (end 170.904 89.118) (width 0.75) (layer "B.Cu") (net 1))
 (segment (start 187.1805 93.4545) (end 185.42 91.694) (width 1) (layer "B.Cu") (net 1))
 (segment (start 178.854 88.608) (end 182.372 85.09) (width 0.75) (layer "B.Cu") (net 1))
 (segment (start 179.324 78.994) (end 179.324 79.502) (width 1) (layer "B.Cu") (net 1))
 (segment (start 178.854 89.118) (end 178.854 88.608) (width 0.75) (layer "B.Cu") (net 1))
 (segment (start 179.334 78.984) (end 179.324 78.994) (width 1) (layer "B.Cu") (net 1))
 (segment (start 185.42 90.932) (end 185.42 87.122) (width 1) (layer "B.Cu") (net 1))
 (segment (start 185.42 80.264) (end 185.42 85.09) (width 1) (layer "B.Cu") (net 1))
 (segment (start 178.9815 79.8445) (end 179.324 79.502) (width 0.75) (layer "B.Cu") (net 1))
 (segment (start 185.42 80.264) (end 183.642 78.486) (width 1) (layer "B.Cu") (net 1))
 (segment (start 182.372 85.09) (end 185.42 85.09) (width 0.75) (layer "B.Cu") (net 1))
 (segment (start 183.642 78.486) (end 180.34 78.486) (width 1) (layer "B.Cu") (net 1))
 (segment (start 185.42 91.694) (end 185.42 90.932) (width 1) (layer "B.Cu") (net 1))
 (segment (start 180.34 78.486) (end 179.324 79.502) (width 1) (layer "B.Cu") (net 1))
 (segment (start 165.862 91.79) (end 167.036 91.79) (width 0.75) (layer "B.Cu") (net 1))
 (segment (start 170.904 89.118) (end 178.854 89.118) (width 0.75) (layer "B.Cu") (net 1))
 (segment (start 167.036 91.79) (end 169.708 89.118) (width 0.75) (layer "B.Cu") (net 1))
 (segment (start 187.1805 93.9995) (end 187.1805 93.4545) (width 1) (layer "B.Cu") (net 1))
 (segment (start 188.214 96.774) (end 189.357 95.631) (width 1) (layer "B.Cu") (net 4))
 (segment (start 187.452 82.55) (end 189.23 80.772) (width 1) (layer "B.Cu") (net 4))
 (segment (start 177.673 95.758) (end 178.355 95.758) (width 1) (layer "B.Cu") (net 4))
 (segment (start 189.357 90.043) (end 187.452 88.138) (width 1) (layer "B.Cu") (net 4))
 (segment (start 178.355 95.758) (end 179.371 96.774) (width 1) (layer "B.Cu") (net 4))
 (segment (start 179.371 96.774) (end 188.214 96.774) (width 1) (layer "B.Cu") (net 4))
 (segment (start 189.23 80.772) (end 190.5 80.772) (width 1) (layer "B.Cu") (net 4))
 (segment (start 189.357 95.631) (end 189.357 90.043) (width 1) (layer "B.Cu") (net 4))
 (segment (start 187.452 88.138) (end 187.452 82.55) (width 1) (layer "B.Cu") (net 4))
 (segment (start 174.117 92.202) (end 177.673 95.758) (width 1) (layer "B.Cu") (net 4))
 (segment (start 173.395 92.202) (end 174.117 92.202) (width 1) (layer "B.Cu") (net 4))
 (segment (start 178.395 92.202) (end 180.303 92.202) (width 1) (layer "B.Cu") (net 9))
 (segment (start 180.303 92.202) (end 182.1005 93.9995) (width 1) (layer "B.Cu") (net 9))
 (segment (start 173.355 95.758) (end 165.894 95.758) (width 1) (layer "B.Cu") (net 12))
 (segment (start 165.894 95.758) (end 165.862 95.79) (width 1) (layer "B.Cu") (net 12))
 (segment (start 181.356 73.406) (end 180.594 74.168) (width 0.75) (layer "B.Cu") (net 7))
 (segment (start 182.88 73.406) (end 181.356 73.406) (width 0.75) (layer "B.Cu") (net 7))
 (segment (start 176.784 72.898) (end 176.784 71.882) (width 0.75) (layer "B.Cu") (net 7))
 (segment (start 180.594 74.168) (end 178.054 74.168) (width 0.75) (layer "B.Cu") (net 7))
 (segment (start 176.784 72.644) (end 176.784 71.882) (width 0.5) (layer "B.Cu") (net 7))
 (segment (start 178.054 74.168) (end 176.784 72.898) (width 0.75) (layer "B.Cu") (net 7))
 (segment (start 185.42 73.406) (end 185.42 71.146) (width 0.75) (layer "B.Cu") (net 8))
 (segment (start 183.922 81.306) (end 182.88 80.264) (width 0.5) (layer "B.Cu") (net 6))
 (segment (start 183.922 83.312) (end 183.922 81.306) (width 0.5) (layer "B.Cu") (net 6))
 (segment (start 182.88 87.122) (end 182.88 88.112) (width 0.5) (layer "B.Cu") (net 2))
 (segment (start 182.88 88.112) (end 183.922 89.154) (width 0.5) (layer "B.Cu") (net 2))
 (segment (start 184.124 69.342) (end 185.859726 69.342) (width 0.75) (layer "B.Cu") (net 5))
 (segment (start 169.672 71.247) (end 171.069 69.85) (width 0.75) (layer "B.Cu") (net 5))
 (segment (start 187.579 73.787) (end 190.5 76.708) (width 0.75) (layer "B.Cu") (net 5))
 (segment (start 182.346 71.12) (end 180.086 71.12) (width 0.75) (layer "B.Cu") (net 5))
 (segment (start 188.849 98.171) (end 166.243 98.171) (width 1) (layer "B.Cu") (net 5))
 (segment (start 182.346 71.12) (end 184.124 69.342) (width 0.75) (layer "B.Cu") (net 5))
 (segment (start 193.548 79.756) (end 193.548 85.344) (width 1) (layer "B.Cu") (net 5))
 (segment (start 166.243 98.171) (end 165.862 97.79) (width 1) (layer "B.Cu") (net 5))
 (segment (start 190.5 77.772) (end 191.564 77.772) (width 1) (layer "B.Cu") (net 5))
 (segment (start 169.672 73.279) (end 169.672 71.247) (width 0.75) (layer "B.Cu") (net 5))
 (segment (start 179.324 71.628) (end 179.324 71.882) (width 0.75) (layer "B.Cu") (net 5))
 (segment (start 168.91 74.523) (end 168.91 74.041) (width 0.75) (layer "B.Cu") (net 5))
 (segment (start 193.548 85.344) (end 190.754 88.138) (width 1) (layer "B.Cu") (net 5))
 (segment (start 190.754 96.266) (end 188.849 98.171) (width 1) (layer "B.Cu") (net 5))
 (segment (start 190.5 76.708) (end 190.5 77.772) (width 0.75) (layer "B.Cu") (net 5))
 (segment (start 171.069 69.85) (end 177.546 69.85) (width 0.75) (layer "B.Cu") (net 5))
 (segment (start 180.086 71.12) (end 179.324 71.882) (width 0.75) (layer "B.Cu") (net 5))
 (segment (start 190.754 88.138) (end 190.754 96.266) (width 1) (layer "B.Cu") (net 5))
 (segment (start 168.91 74.041) (end 169.672 73.279) (width 0.75) (layer "B.Cu") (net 5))
 (segment (start 187.579 71.061274) (end 187.579 73.787) (width 0.75) (layer "B.Cu") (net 5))
 (segment (start 177.546 69.85) (end 179.324 71.628) (width 0.75) (layer "B.Cu") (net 5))
 (segment (start 191.564 77.772) (end 193.548 79.756) (width 1) (layer "B.Cu") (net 5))
 (segment (start 185.859726 69.342) (end 187.579 71.061274) (width 0.75) (layer "B.Cu") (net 5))
 (segment (start 164.459 82.937) (end 164.459 86.735) (width 0.75) (layer "B.Cu") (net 13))
 (segment (start 165.514 87.79) (end 165.862 87.79) (width 0.75) (layer "B.Cu") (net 13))
 (segment (start 164.459 86.735) (end 165.514 87.79) (width 0.75) (layer "B.Cu") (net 13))
 (segment (start 169.164 79.502) (end 167.894 79.502) (width 0.75) (layer "B.Cu") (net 13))
 (segment (start 168.91 79.248) (end 168.91 77.623) (width 0.75) (layer "B.Cu") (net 13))
 (segment (start 169.164 79.502) (end 168.91 79.248) (width 0.75) (layer "B.Cu") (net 13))
 (segment (start 167.894 79.502) (end 164.459 82.937) (width 0.75) (layer "B.Cu") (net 13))
 (segment (start 171.704 79.502) (end 169.164 79.502) (width 0.75) (layer "B.Cu") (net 13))
 (segment (start 168.91 87.884) (end 167.004 89.79) (width 0.75) (layer "B.Cu") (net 16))
 (segment (start 178.054 87.884) (end 168.91 87.884) (width 0.75) (layer "B.Cu") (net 16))
 (segment (start 167.004 89.79) (end 165.862 89.79) (width 0.75) (layer "B.Cu") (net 16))
 (segment (start 180.822 85.116) (end 178.054 87.884) (width 0.75) (layer "B.Cu") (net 16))
 (segment (start 180.822 83.312) (end 180.822 85.116) (width 0.75) (layer "B.Cu") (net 16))
 (segment (start 180.822 89.688) (end 180.086 90.424) (width 0.75) (layer "B.Cu") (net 15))
 (segment (start 167.068 93.79) (end 165.862 93.79) (width 0.75) (layer "B.Cu") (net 15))
 (segment (start 170.434 90.424) (end 167.068 93.79) (width 0.75) (layer "B.Cu") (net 15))
 (segment (start 180.086 90.424) (end 170.434 90.424) (width 0.75) (layer "B.Cu") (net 15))
 (segment (start 180.822 89.154) (end 180.822 89.688) (width 0.75) (layer "B.Cu") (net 15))
 (segment (start 174.244 79.502) (end 171.45 82.296) (width 0.75) (layer "B.Cu") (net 10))
 (segment (start 171.45 82.296) (end 170.789 82.296) (width 0.75) (layer "B.Cu") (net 10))
 (segment (start 165.862 85.79) (end 168.06 85.79) (width 0.75) (layer "B.Cu") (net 17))
 (segment (start 168.06 85.79) (end 168.656 86.386) (width 0.75) (layer "B.Cu") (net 17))
 (segment (start 166.34 83.312) (end 168.63 83.312) (width 0.75) (layer "B.Cu") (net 18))
 (segment (start 168.757 83.286) (end 170.089 84.618) (width 0.75) (layer "B.Cu") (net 18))
 (segment (start 170.089 84.618) (end 170.904 84.618) (width 0.75) (layer "B.Cu") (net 18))
 (segment (start 165.862 83.79) (end 166.34 83.312) (width 0.75) (layer "B.Cu") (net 18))
 (segment (start 168.63 83.312) (end 168.656 83.286) (width 0.75) (layer "B.Cu") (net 18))
 (segment (start 168.656 83.286) (end 168.757 83.286) (width 0.75) (layer "B.Cu") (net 18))
 (segment (start 170.904 84.618) (end 178.854 84.618) (width 0.75) (layer "B.Cu") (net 18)))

